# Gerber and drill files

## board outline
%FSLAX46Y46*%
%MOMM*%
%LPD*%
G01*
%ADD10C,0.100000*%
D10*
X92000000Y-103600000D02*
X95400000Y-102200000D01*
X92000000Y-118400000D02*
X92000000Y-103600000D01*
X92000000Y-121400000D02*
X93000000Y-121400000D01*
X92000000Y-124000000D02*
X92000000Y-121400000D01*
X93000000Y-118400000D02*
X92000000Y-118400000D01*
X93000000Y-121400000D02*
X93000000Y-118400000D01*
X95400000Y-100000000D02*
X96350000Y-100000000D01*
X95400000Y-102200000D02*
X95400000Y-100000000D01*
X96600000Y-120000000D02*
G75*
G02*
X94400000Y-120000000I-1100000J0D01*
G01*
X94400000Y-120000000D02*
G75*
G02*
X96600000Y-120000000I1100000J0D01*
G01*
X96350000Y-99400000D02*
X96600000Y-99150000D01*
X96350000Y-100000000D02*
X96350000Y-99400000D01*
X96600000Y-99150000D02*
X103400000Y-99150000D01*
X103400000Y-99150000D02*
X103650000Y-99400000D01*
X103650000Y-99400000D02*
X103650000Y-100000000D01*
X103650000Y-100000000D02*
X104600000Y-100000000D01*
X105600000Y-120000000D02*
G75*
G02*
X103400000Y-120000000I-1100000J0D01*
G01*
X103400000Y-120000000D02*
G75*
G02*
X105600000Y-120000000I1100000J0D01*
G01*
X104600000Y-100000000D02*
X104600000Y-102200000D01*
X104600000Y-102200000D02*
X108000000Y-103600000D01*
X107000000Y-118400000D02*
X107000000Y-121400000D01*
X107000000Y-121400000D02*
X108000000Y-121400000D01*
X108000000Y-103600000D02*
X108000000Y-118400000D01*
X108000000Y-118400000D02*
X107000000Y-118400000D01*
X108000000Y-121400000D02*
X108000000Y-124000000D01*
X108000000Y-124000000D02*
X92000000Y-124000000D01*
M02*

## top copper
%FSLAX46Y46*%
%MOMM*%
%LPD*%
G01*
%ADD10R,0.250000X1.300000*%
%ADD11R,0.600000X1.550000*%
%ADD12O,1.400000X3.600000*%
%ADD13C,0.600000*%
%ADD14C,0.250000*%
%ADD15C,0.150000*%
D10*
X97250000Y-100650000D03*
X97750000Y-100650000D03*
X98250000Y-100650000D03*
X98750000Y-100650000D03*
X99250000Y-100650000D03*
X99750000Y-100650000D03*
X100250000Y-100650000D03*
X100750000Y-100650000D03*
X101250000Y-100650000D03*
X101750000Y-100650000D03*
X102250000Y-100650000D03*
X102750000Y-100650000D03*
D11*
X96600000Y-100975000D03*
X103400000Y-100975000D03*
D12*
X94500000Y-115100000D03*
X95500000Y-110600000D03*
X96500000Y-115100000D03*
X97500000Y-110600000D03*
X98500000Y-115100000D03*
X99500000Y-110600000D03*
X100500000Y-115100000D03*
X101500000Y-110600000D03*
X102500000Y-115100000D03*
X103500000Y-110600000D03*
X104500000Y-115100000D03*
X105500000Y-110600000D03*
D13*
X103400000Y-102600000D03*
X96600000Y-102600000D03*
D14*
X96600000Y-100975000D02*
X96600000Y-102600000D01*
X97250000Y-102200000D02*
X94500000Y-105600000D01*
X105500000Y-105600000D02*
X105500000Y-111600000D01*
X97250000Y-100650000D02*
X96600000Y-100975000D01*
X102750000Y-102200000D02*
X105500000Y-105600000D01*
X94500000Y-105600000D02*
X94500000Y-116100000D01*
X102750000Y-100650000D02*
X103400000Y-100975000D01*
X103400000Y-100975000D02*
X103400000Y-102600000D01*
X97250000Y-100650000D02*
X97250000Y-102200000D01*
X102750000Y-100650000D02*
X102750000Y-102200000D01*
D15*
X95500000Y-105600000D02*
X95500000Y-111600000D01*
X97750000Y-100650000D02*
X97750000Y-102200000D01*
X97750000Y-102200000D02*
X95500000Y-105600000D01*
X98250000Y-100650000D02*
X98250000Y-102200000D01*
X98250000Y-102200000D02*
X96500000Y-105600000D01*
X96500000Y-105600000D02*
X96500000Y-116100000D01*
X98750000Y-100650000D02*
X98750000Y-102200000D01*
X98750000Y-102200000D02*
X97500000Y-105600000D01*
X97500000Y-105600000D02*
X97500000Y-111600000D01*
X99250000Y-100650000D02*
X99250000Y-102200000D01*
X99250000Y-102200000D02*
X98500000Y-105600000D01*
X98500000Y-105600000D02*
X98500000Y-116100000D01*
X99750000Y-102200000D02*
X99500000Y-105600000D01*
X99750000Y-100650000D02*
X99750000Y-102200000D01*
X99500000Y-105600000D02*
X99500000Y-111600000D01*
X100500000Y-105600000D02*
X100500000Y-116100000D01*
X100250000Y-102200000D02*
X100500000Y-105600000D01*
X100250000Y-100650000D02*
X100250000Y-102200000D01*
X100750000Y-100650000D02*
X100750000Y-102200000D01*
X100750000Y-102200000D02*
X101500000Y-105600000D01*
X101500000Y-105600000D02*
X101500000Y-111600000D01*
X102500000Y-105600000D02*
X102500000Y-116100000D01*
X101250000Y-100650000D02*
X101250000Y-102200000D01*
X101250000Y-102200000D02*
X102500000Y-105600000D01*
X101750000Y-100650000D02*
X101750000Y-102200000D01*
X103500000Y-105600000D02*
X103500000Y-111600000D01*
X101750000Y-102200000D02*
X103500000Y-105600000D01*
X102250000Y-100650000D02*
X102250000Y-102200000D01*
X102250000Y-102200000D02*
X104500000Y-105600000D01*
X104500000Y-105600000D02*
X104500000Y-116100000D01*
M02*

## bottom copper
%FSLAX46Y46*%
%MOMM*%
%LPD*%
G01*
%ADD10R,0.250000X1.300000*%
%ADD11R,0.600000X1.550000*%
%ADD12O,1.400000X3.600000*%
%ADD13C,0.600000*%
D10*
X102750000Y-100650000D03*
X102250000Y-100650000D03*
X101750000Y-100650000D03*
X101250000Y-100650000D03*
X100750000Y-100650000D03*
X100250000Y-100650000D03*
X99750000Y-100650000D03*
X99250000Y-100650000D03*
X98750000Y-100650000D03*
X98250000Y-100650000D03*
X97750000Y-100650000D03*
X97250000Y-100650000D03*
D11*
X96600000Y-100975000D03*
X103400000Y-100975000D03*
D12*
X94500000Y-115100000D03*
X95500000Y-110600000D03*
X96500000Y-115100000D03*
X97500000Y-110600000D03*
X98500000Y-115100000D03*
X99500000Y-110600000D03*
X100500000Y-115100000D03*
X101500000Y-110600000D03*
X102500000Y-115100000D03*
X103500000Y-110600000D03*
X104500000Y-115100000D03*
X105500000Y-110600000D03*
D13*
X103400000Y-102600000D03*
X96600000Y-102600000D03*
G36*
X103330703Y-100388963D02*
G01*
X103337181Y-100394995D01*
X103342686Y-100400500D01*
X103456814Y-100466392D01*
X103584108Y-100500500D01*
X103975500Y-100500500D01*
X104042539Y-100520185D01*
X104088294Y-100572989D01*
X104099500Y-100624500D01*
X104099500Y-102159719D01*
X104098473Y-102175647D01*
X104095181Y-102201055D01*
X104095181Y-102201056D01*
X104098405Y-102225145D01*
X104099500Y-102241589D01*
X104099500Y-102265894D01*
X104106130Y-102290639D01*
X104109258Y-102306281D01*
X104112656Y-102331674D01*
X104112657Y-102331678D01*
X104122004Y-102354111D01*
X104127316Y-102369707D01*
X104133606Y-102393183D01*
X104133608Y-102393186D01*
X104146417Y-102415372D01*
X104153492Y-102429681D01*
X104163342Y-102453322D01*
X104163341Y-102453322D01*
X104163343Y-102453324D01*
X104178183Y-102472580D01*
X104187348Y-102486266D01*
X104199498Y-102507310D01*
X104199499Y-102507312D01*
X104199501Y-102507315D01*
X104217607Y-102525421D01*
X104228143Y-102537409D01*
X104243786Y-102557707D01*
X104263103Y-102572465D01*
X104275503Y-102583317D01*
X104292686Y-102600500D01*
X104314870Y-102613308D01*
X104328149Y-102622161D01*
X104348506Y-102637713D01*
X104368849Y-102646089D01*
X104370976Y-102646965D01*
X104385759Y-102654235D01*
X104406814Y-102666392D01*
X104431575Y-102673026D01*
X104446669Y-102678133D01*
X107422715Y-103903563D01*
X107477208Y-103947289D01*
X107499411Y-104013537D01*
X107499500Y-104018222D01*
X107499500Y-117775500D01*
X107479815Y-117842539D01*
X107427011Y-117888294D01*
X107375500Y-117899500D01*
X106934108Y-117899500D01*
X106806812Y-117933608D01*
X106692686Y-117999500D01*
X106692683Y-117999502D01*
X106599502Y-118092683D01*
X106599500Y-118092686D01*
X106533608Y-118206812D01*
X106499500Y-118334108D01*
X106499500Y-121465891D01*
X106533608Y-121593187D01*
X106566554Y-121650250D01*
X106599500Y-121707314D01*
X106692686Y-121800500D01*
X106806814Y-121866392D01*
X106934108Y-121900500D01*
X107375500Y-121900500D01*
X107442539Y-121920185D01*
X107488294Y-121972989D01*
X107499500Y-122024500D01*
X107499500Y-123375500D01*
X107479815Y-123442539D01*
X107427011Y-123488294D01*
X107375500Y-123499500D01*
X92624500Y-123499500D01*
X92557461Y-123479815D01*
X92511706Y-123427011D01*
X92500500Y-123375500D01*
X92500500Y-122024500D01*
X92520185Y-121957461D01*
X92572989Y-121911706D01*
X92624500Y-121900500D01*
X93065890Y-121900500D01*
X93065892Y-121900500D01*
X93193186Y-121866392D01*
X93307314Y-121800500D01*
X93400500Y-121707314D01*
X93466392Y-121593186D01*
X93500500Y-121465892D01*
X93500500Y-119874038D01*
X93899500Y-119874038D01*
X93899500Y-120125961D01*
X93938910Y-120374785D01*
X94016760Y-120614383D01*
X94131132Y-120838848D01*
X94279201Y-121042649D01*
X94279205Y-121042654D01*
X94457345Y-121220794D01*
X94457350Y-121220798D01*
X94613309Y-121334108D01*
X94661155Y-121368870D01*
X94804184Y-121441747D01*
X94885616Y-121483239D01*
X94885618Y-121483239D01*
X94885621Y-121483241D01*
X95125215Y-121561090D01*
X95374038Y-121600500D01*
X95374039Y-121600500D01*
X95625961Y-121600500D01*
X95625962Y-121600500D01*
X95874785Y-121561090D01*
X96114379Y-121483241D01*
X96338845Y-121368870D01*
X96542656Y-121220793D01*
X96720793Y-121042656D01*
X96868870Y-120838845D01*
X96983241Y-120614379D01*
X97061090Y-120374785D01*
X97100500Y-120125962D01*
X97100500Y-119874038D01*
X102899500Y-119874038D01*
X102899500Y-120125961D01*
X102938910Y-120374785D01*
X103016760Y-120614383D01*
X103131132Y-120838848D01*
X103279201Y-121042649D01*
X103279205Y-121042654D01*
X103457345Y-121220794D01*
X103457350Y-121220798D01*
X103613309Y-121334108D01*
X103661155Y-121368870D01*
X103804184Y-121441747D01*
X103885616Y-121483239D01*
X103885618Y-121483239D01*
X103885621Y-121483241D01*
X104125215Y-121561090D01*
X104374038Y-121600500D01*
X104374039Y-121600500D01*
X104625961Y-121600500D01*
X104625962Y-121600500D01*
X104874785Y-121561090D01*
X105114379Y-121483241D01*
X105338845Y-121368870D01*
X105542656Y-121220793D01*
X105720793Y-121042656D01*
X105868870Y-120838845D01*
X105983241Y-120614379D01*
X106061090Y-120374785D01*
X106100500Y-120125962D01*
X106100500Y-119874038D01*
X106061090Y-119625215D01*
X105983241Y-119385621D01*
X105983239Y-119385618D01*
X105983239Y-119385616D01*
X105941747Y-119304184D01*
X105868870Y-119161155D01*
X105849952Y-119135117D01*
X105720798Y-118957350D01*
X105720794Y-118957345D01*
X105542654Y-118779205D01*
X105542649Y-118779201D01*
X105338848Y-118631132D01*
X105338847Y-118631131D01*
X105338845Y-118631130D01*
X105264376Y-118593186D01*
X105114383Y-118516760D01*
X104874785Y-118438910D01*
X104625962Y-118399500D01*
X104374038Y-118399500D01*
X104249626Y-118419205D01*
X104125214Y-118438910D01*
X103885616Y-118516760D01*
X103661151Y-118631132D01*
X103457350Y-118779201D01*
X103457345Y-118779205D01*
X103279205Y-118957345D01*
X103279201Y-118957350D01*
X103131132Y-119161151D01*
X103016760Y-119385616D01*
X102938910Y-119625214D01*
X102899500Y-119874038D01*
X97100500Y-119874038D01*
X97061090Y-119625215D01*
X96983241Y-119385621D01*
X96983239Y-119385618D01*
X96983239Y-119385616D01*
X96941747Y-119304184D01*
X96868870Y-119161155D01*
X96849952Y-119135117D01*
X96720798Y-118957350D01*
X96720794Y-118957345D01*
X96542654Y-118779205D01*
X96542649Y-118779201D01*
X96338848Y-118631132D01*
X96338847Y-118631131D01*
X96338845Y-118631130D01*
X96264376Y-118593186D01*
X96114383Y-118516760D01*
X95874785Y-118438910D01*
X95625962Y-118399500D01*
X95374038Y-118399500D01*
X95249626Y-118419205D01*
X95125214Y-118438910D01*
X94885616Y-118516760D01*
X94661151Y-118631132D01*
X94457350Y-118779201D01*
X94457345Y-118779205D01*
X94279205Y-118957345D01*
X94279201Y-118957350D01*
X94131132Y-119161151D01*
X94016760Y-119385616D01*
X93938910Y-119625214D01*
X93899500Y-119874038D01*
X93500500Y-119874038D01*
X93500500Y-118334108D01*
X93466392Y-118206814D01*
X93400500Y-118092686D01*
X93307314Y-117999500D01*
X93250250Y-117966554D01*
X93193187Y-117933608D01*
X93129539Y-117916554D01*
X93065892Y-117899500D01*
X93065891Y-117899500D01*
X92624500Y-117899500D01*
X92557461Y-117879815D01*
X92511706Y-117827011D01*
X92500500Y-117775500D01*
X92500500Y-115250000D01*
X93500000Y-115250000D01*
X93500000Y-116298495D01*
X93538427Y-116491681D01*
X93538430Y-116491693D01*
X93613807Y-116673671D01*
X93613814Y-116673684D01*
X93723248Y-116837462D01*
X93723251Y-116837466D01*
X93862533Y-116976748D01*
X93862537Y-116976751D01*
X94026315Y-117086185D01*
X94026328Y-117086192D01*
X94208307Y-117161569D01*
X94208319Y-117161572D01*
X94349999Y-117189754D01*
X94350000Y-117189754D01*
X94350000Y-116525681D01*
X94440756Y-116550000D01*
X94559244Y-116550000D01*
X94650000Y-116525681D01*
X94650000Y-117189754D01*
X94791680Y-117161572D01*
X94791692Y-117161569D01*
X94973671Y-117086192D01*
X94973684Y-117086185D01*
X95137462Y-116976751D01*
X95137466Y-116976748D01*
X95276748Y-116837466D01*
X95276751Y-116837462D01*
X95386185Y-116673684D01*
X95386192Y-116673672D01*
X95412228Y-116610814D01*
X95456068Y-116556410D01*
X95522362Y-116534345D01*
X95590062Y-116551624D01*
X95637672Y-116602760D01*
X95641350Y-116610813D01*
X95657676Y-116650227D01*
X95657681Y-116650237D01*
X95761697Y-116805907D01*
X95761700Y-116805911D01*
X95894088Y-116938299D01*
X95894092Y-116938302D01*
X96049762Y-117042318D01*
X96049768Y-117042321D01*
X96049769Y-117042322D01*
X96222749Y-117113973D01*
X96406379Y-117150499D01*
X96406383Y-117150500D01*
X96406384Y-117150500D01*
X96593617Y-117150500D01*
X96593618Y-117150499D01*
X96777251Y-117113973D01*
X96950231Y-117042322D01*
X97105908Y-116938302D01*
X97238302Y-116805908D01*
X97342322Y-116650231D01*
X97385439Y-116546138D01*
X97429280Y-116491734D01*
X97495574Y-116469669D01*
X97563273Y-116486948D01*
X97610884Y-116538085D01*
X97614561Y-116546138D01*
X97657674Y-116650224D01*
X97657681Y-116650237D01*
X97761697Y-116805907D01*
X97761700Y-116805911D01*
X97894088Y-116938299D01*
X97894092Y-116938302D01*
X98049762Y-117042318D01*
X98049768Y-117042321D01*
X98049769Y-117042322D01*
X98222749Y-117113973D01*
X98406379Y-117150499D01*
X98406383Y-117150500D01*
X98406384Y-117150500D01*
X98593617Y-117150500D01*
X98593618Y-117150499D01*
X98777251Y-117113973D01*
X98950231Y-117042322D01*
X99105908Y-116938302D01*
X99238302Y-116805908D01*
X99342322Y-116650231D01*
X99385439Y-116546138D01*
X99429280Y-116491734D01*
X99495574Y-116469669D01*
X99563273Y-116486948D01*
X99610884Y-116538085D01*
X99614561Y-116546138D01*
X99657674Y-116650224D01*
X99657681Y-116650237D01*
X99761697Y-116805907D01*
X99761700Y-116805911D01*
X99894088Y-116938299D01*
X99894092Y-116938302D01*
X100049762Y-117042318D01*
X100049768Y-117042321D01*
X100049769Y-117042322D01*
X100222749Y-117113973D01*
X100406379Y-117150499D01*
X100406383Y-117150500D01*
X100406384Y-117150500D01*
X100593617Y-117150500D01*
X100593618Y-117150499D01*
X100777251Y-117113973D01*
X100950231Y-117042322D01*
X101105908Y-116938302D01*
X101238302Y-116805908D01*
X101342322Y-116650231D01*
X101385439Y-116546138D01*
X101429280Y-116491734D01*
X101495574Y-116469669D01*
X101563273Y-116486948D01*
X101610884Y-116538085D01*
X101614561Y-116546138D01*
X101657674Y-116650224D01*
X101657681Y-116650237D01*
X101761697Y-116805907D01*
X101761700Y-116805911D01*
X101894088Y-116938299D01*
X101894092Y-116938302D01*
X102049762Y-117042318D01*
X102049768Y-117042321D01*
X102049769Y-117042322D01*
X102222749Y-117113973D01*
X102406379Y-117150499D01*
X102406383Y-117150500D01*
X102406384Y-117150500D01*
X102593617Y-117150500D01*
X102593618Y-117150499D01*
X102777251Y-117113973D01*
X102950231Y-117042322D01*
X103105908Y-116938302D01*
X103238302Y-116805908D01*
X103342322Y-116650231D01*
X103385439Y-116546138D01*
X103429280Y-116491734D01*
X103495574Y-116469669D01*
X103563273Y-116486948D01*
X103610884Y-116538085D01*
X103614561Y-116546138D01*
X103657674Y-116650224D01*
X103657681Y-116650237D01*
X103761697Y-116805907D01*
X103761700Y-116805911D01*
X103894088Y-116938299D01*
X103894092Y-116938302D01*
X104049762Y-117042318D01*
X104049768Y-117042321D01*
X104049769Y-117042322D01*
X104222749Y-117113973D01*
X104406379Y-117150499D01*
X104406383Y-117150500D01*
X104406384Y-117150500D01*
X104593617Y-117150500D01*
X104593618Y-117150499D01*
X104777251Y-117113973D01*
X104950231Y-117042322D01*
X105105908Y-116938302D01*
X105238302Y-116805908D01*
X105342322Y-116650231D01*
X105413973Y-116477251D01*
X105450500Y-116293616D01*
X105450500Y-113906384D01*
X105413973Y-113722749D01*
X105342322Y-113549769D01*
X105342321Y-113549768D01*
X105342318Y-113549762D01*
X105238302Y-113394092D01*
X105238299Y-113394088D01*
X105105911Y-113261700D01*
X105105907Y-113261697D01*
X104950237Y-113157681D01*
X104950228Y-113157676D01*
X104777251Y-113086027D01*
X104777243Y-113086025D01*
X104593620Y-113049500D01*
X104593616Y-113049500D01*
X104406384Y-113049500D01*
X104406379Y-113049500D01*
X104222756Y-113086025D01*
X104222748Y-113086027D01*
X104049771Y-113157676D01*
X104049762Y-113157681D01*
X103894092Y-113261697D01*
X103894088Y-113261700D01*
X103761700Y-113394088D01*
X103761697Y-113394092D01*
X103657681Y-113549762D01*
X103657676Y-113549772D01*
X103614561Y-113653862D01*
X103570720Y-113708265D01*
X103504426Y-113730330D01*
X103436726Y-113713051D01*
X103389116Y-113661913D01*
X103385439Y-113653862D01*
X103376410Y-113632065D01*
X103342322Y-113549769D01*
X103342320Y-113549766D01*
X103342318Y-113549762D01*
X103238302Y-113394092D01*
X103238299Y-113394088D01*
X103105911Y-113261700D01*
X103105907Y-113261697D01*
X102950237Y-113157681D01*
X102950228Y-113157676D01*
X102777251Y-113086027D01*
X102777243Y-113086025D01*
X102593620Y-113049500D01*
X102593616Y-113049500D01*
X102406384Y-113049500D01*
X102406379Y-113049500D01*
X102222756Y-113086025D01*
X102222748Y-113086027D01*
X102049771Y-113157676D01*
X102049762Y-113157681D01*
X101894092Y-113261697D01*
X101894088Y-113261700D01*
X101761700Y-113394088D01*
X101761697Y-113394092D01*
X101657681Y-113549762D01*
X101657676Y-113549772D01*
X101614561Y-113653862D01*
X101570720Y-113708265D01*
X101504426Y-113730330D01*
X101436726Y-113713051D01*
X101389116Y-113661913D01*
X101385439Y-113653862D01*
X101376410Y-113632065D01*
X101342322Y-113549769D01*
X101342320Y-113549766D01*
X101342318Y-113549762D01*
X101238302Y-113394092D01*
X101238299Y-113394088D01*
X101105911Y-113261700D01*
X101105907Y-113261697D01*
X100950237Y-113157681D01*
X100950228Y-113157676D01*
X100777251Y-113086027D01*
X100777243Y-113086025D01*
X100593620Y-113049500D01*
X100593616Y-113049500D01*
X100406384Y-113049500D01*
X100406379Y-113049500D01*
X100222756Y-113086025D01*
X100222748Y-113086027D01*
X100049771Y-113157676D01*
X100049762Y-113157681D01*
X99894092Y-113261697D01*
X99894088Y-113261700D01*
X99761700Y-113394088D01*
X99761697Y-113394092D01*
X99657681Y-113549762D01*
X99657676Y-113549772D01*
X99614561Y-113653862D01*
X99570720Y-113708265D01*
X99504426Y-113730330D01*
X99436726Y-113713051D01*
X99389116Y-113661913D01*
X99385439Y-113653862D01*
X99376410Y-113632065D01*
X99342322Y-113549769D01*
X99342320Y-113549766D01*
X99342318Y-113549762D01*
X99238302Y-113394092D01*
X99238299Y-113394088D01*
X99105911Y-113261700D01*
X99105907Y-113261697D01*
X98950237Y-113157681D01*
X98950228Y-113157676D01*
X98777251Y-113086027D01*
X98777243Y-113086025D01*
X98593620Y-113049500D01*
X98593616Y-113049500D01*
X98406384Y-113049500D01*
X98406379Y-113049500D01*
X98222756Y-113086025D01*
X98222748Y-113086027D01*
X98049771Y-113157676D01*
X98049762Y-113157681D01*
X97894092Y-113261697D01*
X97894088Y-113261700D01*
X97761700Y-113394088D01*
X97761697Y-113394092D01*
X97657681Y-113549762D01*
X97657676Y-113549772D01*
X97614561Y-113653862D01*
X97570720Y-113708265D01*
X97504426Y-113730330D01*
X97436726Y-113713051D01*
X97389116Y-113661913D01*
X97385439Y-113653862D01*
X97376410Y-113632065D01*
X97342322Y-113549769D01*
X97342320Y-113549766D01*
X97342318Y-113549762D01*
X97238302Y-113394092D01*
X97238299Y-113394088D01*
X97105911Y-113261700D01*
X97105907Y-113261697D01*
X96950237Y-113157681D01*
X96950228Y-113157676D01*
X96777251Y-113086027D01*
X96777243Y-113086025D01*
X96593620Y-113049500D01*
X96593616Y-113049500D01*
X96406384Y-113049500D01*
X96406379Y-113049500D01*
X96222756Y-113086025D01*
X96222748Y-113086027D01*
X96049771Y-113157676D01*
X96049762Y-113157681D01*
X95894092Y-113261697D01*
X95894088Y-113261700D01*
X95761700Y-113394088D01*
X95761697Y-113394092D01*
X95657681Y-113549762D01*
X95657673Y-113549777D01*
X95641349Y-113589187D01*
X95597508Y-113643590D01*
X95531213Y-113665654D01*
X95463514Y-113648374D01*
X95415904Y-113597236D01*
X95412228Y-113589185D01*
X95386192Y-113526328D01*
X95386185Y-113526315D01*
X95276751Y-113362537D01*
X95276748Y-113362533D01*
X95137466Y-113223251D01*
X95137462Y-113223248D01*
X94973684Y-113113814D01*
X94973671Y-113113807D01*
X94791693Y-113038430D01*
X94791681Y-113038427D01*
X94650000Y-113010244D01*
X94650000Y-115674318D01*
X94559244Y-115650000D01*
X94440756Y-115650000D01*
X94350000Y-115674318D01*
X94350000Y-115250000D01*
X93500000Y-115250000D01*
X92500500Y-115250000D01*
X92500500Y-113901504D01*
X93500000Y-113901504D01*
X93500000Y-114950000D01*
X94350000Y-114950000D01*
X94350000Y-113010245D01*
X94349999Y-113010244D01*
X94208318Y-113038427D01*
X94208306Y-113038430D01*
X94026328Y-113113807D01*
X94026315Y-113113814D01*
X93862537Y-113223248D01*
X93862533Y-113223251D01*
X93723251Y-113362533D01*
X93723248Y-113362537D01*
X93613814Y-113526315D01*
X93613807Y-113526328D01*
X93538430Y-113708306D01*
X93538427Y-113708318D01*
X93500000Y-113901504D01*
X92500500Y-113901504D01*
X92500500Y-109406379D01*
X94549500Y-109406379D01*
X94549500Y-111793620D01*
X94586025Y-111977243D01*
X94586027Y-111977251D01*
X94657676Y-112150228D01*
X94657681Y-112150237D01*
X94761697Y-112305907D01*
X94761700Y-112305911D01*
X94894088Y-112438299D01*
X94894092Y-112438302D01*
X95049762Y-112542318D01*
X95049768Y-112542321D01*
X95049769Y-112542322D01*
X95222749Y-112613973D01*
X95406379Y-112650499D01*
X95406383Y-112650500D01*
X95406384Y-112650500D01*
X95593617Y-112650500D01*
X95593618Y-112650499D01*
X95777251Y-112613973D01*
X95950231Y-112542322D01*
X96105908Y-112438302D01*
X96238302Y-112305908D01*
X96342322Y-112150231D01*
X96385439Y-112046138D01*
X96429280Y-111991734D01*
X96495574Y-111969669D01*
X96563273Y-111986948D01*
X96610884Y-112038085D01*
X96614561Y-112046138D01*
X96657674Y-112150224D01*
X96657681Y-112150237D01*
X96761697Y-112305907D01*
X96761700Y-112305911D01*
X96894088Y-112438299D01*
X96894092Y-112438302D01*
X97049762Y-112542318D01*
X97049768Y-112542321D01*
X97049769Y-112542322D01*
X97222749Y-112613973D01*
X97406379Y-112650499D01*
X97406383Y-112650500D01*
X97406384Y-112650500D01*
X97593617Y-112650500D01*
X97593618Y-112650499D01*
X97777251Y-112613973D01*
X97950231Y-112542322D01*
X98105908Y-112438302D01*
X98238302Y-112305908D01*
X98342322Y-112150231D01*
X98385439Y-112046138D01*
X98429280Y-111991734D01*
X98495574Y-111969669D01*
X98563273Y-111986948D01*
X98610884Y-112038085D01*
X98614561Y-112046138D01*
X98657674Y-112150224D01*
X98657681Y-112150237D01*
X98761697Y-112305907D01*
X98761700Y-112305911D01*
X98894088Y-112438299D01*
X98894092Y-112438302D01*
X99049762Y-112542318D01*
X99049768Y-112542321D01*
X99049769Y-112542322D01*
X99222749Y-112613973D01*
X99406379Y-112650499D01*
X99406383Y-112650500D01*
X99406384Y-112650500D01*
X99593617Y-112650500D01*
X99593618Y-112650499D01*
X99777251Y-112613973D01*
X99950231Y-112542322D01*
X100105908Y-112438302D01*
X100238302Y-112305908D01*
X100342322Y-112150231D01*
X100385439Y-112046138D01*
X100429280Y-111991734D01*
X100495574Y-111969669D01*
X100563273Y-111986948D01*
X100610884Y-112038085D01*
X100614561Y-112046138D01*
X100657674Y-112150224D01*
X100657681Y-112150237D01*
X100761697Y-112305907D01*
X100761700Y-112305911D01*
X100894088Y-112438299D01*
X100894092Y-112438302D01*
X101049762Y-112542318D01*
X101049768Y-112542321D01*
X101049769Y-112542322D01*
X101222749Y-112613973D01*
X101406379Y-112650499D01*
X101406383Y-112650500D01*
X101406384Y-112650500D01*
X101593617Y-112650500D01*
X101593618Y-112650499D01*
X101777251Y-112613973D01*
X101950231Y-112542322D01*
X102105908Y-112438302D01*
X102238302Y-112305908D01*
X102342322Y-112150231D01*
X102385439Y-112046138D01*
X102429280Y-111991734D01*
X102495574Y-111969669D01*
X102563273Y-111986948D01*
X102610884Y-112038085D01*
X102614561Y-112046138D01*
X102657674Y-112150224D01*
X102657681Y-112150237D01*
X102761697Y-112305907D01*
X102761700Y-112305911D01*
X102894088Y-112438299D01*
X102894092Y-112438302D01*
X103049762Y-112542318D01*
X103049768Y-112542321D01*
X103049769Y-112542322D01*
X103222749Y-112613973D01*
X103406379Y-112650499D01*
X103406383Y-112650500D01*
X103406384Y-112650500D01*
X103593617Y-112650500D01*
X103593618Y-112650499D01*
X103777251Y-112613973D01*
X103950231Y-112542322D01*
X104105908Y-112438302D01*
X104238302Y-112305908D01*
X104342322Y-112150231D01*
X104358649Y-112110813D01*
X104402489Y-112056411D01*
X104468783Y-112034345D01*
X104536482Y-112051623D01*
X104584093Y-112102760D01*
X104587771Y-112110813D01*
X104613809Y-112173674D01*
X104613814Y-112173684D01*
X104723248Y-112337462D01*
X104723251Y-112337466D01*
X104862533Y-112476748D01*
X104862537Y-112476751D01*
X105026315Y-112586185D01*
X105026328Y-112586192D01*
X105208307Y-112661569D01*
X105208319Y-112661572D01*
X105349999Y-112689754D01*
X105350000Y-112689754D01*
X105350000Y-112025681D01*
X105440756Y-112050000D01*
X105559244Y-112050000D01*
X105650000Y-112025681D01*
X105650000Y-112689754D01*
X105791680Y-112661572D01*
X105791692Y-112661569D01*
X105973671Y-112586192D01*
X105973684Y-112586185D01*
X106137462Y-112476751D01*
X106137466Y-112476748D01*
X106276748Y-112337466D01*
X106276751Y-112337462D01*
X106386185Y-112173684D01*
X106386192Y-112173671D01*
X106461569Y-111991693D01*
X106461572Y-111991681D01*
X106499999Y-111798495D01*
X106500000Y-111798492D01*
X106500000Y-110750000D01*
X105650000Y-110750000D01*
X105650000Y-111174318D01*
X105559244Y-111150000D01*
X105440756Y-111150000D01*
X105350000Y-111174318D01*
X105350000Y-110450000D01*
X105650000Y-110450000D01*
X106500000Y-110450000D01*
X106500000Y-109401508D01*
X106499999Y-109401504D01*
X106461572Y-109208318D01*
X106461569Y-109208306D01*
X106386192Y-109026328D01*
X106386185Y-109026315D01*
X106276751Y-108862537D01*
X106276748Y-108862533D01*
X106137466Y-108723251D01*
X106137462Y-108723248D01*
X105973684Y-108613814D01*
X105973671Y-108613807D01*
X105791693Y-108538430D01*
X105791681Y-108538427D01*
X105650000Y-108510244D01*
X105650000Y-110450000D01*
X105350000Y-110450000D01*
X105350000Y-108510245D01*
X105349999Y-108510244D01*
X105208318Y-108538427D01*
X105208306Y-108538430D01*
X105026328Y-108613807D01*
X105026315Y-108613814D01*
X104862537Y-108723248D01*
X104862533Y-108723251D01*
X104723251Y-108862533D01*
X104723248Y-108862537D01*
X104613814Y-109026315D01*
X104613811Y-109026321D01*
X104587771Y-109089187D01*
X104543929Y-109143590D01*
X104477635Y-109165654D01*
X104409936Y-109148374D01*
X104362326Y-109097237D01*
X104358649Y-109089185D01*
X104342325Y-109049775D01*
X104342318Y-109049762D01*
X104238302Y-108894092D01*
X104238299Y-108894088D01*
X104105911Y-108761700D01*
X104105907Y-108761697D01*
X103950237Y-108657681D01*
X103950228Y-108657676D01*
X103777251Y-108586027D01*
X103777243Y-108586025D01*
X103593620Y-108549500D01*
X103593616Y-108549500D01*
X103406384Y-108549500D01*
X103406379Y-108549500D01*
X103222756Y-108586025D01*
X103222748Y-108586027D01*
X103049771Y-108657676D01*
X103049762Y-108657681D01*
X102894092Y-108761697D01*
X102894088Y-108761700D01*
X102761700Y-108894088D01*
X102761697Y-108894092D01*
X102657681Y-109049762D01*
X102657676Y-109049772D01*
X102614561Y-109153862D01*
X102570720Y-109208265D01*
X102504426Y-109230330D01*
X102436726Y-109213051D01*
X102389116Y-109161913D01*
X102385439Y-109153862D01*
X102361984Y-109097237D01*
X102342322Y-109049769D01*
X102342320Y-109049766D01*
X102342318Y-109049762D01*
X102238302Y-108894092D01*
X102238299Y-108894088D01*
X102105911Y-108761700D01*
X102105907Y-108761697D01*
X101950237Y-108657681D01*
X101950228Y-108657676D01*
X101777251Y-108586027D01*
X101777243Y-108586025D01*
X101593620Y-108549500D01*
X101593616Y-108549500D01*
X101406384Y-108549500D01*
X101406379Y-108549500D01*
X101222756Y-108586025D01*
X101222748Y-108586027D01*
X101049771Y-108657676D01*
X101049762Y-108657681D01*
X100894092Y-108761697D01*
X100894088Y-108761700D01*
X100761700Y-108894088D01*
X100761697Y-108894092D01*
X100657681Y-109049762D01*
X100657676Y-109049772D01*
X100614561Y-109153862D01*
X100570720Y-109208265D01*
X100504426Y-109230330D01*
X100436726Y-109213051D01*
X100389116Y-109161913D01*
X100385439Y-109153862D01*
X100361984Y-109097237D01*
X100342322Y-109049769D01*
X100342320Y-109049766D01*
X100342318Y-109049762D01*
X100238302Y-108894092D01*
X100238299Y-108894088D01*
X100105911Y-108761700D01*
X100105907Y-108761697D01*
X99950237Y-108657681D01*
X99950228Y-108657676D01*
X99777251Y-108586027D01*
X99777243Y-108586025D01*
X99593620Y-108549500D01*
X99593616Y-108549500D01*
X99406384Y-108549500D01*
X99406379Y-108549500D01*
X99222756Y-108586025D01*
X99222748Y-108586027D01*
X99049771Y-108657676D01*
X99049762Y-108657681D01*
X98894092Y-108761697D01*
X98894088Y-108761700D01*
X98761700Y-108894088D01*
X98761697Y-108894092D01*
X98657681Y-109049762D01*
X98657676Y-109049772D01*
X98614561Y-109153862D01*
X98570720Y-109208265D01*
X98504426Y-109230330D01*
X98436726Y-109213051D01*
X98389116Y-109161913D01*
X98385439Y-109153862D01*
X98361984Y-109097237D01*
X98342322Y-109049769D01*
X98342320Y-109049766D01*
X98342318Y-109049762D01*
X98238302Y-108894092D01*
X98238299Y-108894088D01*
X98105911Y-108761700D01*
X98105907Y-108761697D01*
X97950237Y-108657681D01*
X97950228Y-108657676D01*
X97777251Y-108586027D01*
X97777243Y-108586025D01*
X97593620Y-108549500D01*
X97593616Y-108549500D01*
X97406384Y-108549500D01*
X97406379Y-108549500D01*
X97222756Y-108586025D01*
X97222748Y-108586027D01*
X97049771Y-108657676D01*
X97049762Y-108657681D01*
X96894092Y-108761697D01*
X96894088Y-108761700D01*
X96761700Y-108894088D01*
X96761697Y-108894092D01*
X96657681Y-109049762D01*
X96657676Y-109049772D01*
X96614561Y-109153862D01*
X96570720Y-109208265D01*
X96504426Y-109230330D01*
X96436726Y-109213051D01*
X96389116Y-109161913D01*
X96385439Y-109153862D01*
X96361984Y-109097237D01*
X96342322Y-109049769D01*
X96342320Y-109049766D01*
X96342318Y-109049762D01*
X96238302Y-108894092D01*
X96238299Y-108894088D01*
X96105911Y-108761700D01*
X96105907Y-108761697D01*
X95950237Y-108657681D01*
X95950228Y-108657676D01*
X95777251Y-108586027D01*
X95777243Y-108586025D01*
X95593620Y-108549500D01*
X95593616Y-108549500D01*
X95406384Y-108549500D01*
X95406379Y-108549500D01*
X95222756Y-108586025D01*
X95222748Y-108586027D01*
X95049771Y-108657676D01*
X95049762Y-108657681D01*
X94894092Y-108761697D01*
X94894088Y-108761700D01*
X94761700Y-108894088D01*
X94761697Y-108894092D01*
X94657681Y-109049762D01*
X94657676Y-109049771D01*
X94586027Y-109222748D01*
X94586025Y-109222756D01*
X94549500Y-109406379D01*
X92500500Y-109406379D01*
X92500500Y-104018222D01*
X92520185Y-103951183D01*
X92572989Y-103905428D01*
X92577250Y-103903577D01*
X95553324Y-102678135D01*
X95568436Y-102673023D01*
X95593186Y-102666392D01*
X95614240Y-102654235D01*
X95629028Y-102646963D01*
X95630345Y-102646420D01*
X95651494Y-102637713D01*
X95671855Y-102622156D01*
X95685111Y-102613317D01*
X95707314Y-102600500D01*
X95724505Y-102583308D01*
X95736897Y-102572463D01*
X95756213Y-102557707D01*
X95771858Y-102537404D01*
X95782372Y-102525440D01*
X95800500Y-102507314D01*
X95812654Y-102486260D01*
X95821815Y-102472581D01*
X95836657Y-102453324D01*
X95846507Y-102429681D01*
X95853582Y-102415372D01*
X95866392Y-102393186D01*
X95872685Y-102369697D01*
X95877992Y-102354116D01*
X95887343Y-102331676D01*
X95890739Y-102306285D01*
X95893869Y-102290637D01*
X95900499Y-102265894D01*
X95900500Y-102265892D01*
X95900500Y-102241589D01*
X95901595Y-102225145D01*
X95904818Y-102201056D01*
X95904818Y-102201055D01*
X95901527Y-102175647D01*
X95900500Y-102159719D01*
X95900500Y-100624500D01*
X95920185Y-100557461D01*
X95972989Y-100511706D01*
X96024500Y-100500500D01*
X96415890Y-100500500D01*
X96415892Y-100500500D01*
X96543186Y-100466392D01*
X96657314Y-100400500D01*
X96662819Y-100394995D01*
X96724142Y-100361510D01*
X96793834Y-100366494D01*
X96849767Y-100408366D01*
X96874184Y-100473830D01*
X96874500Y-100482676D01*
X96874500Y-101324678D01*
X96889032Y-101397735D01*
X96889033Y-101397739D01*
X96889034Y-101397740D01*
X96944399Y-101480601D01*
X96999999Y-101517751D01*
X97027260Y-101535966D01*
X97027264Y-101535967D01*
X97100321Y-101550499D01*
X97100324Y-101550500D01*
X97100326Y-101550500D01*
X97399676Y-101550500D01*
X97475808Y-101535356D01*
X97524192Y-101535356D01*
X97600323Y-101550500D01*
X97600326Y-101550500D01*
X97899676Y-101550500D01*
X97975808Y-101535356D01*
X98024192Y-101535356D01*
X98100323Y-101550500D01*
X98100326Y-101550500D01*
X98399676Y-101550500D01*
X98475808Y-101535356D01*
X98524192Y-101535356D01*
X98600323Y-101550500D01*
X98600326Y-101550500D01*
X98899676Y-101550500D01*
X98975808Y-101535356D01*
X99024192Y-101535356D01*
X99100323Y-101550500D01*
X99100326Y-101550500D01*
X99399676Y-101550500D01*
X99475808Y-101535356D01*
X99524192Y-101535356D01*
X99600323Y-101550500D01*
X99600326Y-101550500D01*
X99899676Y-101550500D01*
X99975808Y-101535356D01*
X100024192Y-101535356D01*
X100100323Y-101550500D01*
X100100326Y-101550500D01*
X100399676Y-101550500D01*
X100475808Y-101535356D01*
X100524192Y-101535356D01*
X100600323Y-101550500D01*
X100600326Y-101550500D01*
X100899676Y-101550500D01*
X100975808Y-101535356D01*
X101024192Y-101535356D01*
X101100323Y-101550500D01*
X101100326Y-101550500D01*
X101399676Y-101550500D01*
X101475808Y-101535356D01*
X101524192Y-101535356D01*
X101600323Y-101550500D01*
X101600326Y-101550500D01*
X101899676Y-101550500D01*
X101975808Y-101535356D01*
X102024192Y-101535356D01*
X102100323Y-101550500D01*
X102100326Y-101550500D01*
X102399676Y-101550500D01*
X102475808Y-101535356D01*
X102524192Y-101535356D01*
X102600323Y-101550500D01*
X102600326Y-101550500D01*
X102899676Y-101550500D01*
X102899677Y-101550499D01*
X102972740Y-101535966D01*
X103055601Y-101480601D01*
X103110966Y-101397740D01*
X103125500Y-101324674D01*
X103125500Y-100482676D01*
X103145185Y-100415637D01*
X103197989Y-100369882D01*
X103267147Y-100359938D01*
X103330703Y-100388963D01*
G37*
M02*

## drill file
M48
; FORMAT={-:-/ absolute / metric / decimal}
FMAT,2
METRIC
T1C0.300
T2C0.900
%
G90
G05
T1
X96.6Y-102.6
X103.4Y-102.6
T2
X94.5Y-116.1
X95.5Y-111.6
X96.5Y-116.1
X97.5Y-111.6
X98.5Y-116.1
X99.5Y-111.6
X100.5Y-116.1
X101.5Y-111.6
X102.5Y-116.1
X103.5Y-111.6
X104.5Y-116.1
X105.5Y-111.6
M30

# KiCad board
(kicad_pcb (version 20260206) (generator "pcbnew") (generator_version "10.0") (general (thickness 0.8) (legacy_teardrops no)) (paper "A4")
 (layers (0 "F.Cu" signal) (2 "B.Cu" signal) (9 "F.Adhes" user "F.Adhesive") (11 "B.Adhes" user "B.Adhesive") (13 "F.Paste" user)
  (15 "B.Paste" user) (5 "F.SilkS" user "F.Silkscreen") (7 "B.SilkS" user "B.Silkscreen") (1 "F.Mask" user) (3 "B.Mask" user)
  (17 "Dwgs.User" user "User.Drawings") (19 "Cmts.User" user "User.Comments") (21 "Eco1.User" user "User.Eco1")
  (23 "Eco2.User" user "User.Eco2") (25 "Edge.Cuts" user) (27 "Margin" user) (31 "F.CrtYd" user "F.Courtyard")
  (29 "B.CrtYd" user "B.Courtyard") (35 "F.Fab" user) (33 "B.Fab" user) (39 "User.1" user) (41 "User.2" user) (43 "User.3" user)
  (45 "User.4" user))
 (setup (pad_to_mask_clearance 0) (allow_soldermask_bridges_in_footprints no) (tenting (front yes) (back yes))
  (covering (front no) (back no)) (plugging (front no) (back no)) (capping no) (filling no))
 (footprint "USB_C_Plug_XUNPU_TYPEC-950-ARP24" (layer "F.Cu") (at 100 100)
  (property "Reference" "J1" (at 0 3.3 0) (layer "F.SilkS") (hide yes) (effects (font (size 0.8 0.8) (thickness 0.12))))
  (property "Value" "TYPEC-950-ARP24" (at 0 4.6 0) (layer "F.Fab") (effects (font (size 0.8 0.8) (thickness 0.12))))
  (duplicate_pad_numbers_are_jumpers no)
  (pad "A1" smd rect (at -2.75 0.65) (size 0.25 1.3) (layers "F.Cu" "F.Mask" "F.Paste") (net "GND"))
  (pad "A2" smd rect (at -2.25 0.65) (size 0.25 1.3) (layers "F.Cu" "F.Mask" "F.Paste") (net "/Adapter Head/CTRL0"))
  (pad "A3" smd rect (at -1.75 0.65) (size 0.25 1.3) (layers "F.Cu" "F.Mask" "F.Paste") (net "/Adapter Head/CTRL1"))
  (pad "A4" smd rect (at -1.25 0.65) (size 0.25 1.3) (layers "F.Cu" "F.Mask" "F.Paste") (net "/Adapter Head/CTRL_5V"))
  (pad "A5" smd rect (at -0.75 0.65) (size 0.25 1.3) (layers "F.Cu" "F.Mask" "F.Paste") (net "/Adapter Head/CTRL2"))
  (pad "A6" smd rect (at -0.25 0.65) (size 0.25 1.3) (layers "F.Cu" "F.Mask" "F.Paste") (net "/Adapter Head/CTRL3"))
  (pad "A7" smd rect (at 0.25 0.65) (size 0.25 1.3) (layers "F.Cu" "F.Mask" "F.Paste") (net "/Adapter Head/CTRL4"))
  (pad "A8" smd rect (at 0.75 0.65) (size 0.25 1.3) (layers "F.Cu" "F.Mask" "F.Paste") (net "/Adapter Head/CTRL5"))
  (pad "A9" smd rect (at 1.25 0.65) (size 0.25 1.3) (layers "F.Cu" "F.Mask" "F.Paste") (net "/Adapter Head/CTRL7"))
  (pad "A10" smd rect (at 1.75 0.65) (size 0.25 1.3) (layers "F.Cu" "F.Mask" "F.Paste") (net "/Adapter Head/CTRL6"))
  (pad "A11" smd rect (at 2.25 0.65) (size 0.25 1.3) (layers "F.Cu" "F.Mask" "F.Paste") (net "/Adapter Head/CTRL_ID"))
  (pad "A12" smd rect (at 2.75 0.65) (size 0.25 1.3) (layers "F.Cu" "F.Mask" "F.Paste") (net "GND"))
  (pad "B1" smd rect (at 2.75 0.65) (size 0.25 1.3) (layers "B.Cu" "B.Mask" "B.Paste") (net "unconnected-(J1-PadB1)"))
  (pad "B2" smd rect (at 2.25 0.65) (size 0.25 1.3) (layers "B.Cu" "B.Mask" "B.Paste") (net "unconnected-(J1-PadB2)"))
  (pad "B3" smd rect (at 1.75 0.65) (size 0.25 1.3) (layers "B.Cu" "B.Mask" "B.Paste") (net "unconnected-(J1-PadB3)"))
  (pad "B4" smd rect (at 1.25 0.65) (size 0.25 1.3) (layers "B.Cu" "B.Mask" "B.Paste") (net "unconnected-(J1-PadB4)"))
  (pad "B5" smd rect (at 0.75 0.65) (size 0.25 1.3) (layers "B.Cu" "B.Mask" "B.Paste") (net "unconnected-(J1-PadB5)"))
  (pad "B6" smd rect (at 0.25 0.65) (size 0.25 1.3) (layers "B.Cu" "B.Mask" "B.Paste") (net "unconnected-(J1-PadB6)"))
  (pad "B7" smd rect (at -0.25 0.65) (size 0.25 1.3) (layers "B.Cu" "B.Mask" "B.Paste") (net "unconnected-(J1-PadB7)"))
  (pad "B8" smd rect (at -0.75 0.65) (size 0.25 1.3) (layers "B.Cu" "B.Mask" "B.Paste") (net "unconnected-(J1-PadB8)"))
  (pad "B9" smd rect (at -1.25 0.65) (size 0.25 1.3) (layers "B.Cu" "B.Mask" "B.Paste") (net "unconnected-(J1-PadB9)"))
  (pad "B10" smd rect (at -1.75 0.65) (size 0.25 1.3) (layers "B.Cu" "B.Mask" "B.Paste") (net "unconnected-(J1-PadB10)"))
  (pad "B11" smd rect (at -2.25 0.65) (size 0.25 1.3) (layers "B.Cu" "B.Mask" "B.Paste") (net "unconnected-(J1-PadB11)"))
  (pad "B12" smd rect (at -2.75 0.65) (size 0.25 1.3) (layers "B.Cu" "B.Mask" "B.Paste") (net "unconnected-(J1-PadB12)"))
  (pad "SH" smd rect (at -3.4 0.975) (size 0.6 1.55) (layers "F.Cu" "F.Mask" "F.Paste") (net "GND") (zone_connect 2))
  (pad "SH" smd rect (at -3.4 0.975) (size 0.6 1.55) (layers "B.Cu" "B.Mask" "B.Paste") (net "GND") (zone_connect 2))
  (pad "SH" smd rect (at 3.4 0.975) (size 0.6 1.55) (layers "F.Cu" "F.Mask" "F.Paste") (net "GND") (zone_connect 2))
  (pad "SH" smd rect (at 3.4 0.975) (size 0.6 1.55) (layers "B.Cu" "B.Mask" "B.Paste") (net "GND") (zone_connect 2)))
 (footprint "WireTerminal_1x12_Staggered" (layer "F.Cu") (at 100 111.6)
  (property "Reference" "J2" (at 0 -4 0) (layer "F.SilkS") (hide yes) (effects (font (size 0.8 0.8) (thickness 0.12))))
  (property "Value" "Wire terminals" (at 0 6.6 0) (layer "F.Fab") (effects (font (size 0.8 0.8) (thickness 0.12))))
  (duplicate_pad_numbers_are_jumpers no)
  (pad "1" thru_hole oval (at -5.5 4.5) (size 1.4 3.6) (drill 0.9 (offset 0 -1)) (layers "*.Cu" "*.Mask") (remove_unused_layers no)
   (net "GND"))
  (pad "2" thru_hole oval (at -4.5 0) (size 1.4 3.6) (drill 0.9 (offset 0 -1)) (layers "*.Cu" "*.Mask") (remove_unused_layers no)
   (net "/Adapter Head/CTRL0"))
  (pad "3" thru_hole oval (at -3.5 4.5) (size 1.4 3.6) (drill 0.9 (offset 0 -1)) (layers "*.Cu" "*.Mask") (remove_unused_layers no)
   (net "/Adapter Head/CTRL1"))
  (pad "4" thru_hole oval (at -2.5 0) (size 1.4 3.6) (drill 0.9 (offset 0 -1)) (layers "*.Cu" "*.Mask") (remove_unused_layers no)
   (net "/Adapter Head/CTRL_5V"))
  (pad "5" thru_hole oval (at -1.5 4.5) (size 1.4 3.6) (drill 0.9 (offset 0 -1)) (layers "*.Cu" "*.Mask") (remove_unused_layers no)
   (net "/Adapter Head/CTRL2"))
  (pad "6" thru_hole oval (at -0.5 0) (size 1.4 3.6) (drill 0.9 (offset 0 -1)) (layers "*.Cu" "*.Mask") (remove_unused_layers no)
   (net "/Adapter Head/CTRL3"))
  (pad "7" thru_hole oval (at 0.5 4.5) (size 1.4 3.6) (drill 0.9 (offset 0 -1)) (layers "*.Cu" "*.Mask") (remove_unused_layers no)
   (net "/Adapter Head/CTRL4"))
  (pad "8" thru_hole oval (at 1.5 0) (size 1.4 3.6) (drill 0.9 (offset 0 -1)) (layers "*.Cu" "*.Mask") (remove_unused_layers no)
   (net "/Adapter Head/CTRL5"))
  (pad "9" thru_hole oval (at 2.5 4.5) (size 1.4 3.6) (drill 0.9 (offset 0 -1)) (layers "*.Cu" "*.Mask") (remove_unused_layers no)
   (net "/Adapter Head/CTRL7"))
  (pad "10" thru_hole oval (at 3.5 0) (size 1.4 3.6) (drill 0.9 (offset 0 -1)) (layers "*.Cu" "*.Mask") (remove_unused_layers no)
   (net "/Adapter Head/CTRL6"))
  (pad "11" thru_hole oval (at 4.5 4.5) (size 1.4 3.6) (drill 0.9 (offset 0 -1)) (layers "*.Cu" "*.Mask") (remove_unused_layers no)
   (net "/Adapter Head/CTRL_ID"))
  (pad "12" thru_hole oval (at 5.5 0) (size 1.4 3.6) (drill 0.9 (offset 0 -1)) (layers "*.Cu" "*.Mask") (remove_unused_layers no)
   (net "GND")))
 (gr_line (start 92 103.6) (end 95.4 102.2) (stroke (width 0.1) (type default)) (layer "Edge.Cuts"))
 (gr_line (start 92 118.4) (end 92 103.6) (stroke (width 0.1) (type default)) (layer "Edge.Cuts"))
 (gr_line (start 92 121.4) (end 93 121.4) (stroke (width 0.1) (type default)) (layer "Edge.Cuts"))
 (gr_line (start 92 124) (end 92 121.4) (stroke (width 0.1) (type default)) (layer "Edge.Cuts"))
 (gr_line (start 93 118.4) (end 92 118.4) (stroke (width 0.1) (type default)) (layer "Edge.Cuts"))
 (gr_line (start 93 121.4) (end 93 118.4) (stroke (width 0.1) (type default)) (layer "Edge.Cuts"))
 (gr_line (start 95.4 100) (end 96.35 100) (stroke (width 0.1) (type default)) (layer "Edge.Cuts"))
 (gr_line (start 95.4 102.2) (end 95.4 100) (stroke (width 0.1) (type default)) (layer "Edge.Cuts"))
 (gr_circle (center 95.5 120) (end 96.6 120) (stroke (width 0.1) (type default)) (fill no) (layer "Edge.Cuts"))
 (gr_line (start 96.35 99.4) (end 96.6 99.15) (stroke (width 0.1) (type default)) (layer "Edge.Cuts"))
 (gr_line (start 96.35 100) (end 96.35 99.4) (stroke (width 0.1) (type default)) (layer "Edge.Cuts"))
 (gr_line (start 96.6 99.15) (end 103.4 99.15) (stroke (width 0.1) (type default)) (layer "Edge.Cuts"))
 (gr_line (start 103.4 99.15) (end 103.65 99.4) (stroke (width 0.1) (type default)) (layer "Edge.Cuts"))
 (gr_line (start 103.65 99.4) (end 103.65 100) (stroke (width 0.1) (type default)) (layer "Edge.Cuts"))
 (gr_line (start 103.65 100) (end 104.6 100) (stroke (width 0.1) (type default)) (layer "Edge.Cuts"))
 (gr_circle (center 104.5 120) (end 105.6 120) (stroke (width 0.1) (type default)) (fill no) (layer "Edge.Cuts"))
 (gr_line (start 104.6 100) (end 104.6 102.2) (stroke (width 0.1) (type default)) (layer "Edge.Cuts"))
 (gr_line (start 104.6 102.2) (end 108 103.6) (stroke (width 0.1) (type default)) (layer "Edge.Cuts"))
 (gr_line (start 107 118.4) (end 107 121.4) (stroke (width 0.1) (type default)) (layer "Edge.Cuts"))
 (gr_line (start 107 121.4) (end 108 121.4) (stroke (width 0.1) (type default)) (layer "Edge.Cuts"))
 (gr_line (start 108 103.6) (end 108 118.4) (stroke (width 0.1) (type default)) (layer "Edge.Cuts"))
 (gr_line (start 108 118.4) (end 107 118.4) (stroke (width 0.1) (type default)) (layer "Edge.Cuts"))
 (gr_line (start 108 121.4) (end 108 124) (stroke (width 0.1) (type default)) (layer "Edge.Cuts"))
 (gr_line (start 108 124) (end 92 124) (stroke (width 0.1) (type default)) (layer "Edge.Cuts"))
 (segment (start 96.6 100.975) (end 96.6 102.6) (width 0.25) (layer "F.Cu") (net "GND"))
 (segment (start 97.25 102.2) (end 94.5 105.6) (width 0.25) (layer "F.Cu") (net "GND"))
 (segment (start 105.5 105.6) (end 105.5 111.6) (width 0.25) (layer "F.Cu") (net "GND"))
 (segment (start 97.25 100.65) (end 96.6 100.975) (width 0.25) (layer "F.Cu") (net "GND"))
 (segment (start 102.75 102.2) (end 105.5 105.6) (width 0.25) (layer "F.Cu") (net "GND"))
 (segment (start 94.5 105.6) (end 94.5 116.1) (width 0.25) (layer "F.Cu") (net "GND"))
 (segment (start 102.75 100.65) (end 103.4 100.975) (width 0.25) (layer "F.Cu") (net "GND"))
 (segment (start 103.4 100.975) (end 103.4 102.6) (width 0.25) (layer "F.Cu") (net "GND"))
 (segment (start 97.25 100.65) (end 97.25 102.2) (width 0.25) (layer "F.Cu") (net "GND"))
 (segment (start 102.75 100.65) (end 102.75 102.2) (width 0.25) (layer "F.Cu") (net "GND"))
 (via (at 103.4 102.6) (size 0.6) (drill 0.3) (layers "F.Cu" "B.Cu") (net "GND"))
 (via (at 96.6 102.6) (size 0.6) (drill 0.3) (layers "F.Cu" "B.Cu") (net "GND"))
 (segment (start 95.5 105.6) (end 95.5 111.6) (width 0.15) (layer "F.Cu") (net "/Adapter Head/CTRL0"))
 (segment (start 97.75 100.65) (end 97.75 102.2) (width 0.15) (layer "F.Cu") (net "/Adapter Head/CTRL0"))
 (segment (start 97.75 102.2) (end 95.5 105.6) (width 0.15) (layer "F.Cu") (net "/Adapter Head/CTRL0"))
 (segment (start 98.25 100.65) (end 98.25 102.2) (width 0.15) (layer "F.Cu") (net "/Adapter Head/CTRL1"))
 (segment (start 98.25 102.2) (end 96.5 105.6) (width 0.15) (layer "F.Cu") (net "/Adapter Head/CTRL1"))
 (segment (start 96.5 105.6) (end 96.5 116.1) (width 0.15) (layer "F.Cu") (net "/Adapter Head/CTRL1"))
 (segment (start 98.75 100.65) (end 98.75 102.2) (width 0.15) (layer "F.Cu") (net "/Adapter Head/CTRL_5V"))
 (segment (start 98.75 102.2) (end 97.5 105.6) (width 0.15) (layer "F.Cu") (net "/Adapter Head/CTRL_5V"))
 (segment (start 97.5 105.6) (end 97.5 111.6) (width 0.15) (layer "F.Cu") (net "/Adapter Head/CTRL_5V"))
 (segment (start 99.25 100.65) (end 99.25 102.2) (width 0.15) (layer "F.Cu") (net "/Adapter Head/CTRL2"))
 (segment (start 99.25 102.2) (end 98.5 105.6) (width 0.15) (layer "F.Cu") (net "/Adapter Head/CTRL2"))
 (segment (start 98.5 105.6) (end 98.5 116.1) (width 0.15) (layer "F.Cu") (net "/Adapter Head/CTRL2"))
 (segment (start 99.75 102.2) (end 99.5 105.6) (width 0.15) (layer "F.Cu") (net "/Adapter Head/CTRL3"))
 (segment (start 99.75 100.65) (end 99.75 102.2) (width 0.15) (layer "F.Cu") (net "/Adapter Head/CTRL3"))
 (segment (start 99.5 105.6) (end 99.5 111.6) (width 0.15) (layer "F.Cu") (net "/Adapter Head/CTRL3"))
 (segment (start 100.5 105.6) (end 100.5 116.1) (width 0.15) (layer "F.Cu") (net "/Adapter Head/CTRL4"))
 (segment (start 100.25 102.2) (end 100.5 105.6) (width 0.15) (layer "F.Cu") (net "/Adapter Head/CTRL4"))
 (segment (start 100.25 100.65) (end 100.25 102.2) (width 0.15) (layer "F.Cu") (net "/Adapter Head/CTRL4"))
 (segment (start 100.75 100.65) (end 100.75 102.2) (width 0.15) (layer "F.Cu") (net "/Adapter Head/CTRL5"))
 (segment (start 100.75 102.2) (end 101.5 105.6) (width 0.15) (layer "F.Cu") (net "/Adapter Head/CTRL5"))
 (segment (start 101.5 105.6) (end 101.5 111.6) (width 0.15) (layer "F.Cu") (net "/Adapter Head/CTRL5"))
 (segment (start 102.5 105.6) (end 102.5 116.1) (width 0.15) (layer "F.Cu") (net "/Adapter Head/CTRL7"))
 (segment (start 101.25 100.65) (end 101.25 102.2) (width 0.15) (layer "F.Cu") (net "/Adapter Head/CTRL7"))
 (segment (start 101.25 102.2) (end 102.5 105.6) (width 0.15) (layer "F.Cu") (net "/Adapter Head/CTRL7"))
 (segment (start 101.75 100.65) (end 101.75 102.2) (width 0.15) (layer "F.Cu") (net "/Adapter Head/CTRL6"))
 (segment (start 103.5 105.6) (end 103.5 111.6) (width 0.15) (layer "F.Cu") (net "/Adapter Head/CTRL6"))
 (segment (start 101.75 102.2) (end 103.5 105.6) (width 0.15) (layer "F.Cu") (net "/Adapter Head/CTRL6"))
 (segment (start 102.25 100.65) (end 102.25 102.2) (width 0.15) (layer "F.Cu") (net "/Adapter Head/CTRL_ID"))
 (segment (start 102.25 102.2) (end 104.5 105.6) (width 0.15) (layer "F.Cu") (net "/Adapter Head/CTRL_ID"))
 (segment (start 104.5 105.6) (end 104.5 116.1) (width 0.15) (layer "F.Cu") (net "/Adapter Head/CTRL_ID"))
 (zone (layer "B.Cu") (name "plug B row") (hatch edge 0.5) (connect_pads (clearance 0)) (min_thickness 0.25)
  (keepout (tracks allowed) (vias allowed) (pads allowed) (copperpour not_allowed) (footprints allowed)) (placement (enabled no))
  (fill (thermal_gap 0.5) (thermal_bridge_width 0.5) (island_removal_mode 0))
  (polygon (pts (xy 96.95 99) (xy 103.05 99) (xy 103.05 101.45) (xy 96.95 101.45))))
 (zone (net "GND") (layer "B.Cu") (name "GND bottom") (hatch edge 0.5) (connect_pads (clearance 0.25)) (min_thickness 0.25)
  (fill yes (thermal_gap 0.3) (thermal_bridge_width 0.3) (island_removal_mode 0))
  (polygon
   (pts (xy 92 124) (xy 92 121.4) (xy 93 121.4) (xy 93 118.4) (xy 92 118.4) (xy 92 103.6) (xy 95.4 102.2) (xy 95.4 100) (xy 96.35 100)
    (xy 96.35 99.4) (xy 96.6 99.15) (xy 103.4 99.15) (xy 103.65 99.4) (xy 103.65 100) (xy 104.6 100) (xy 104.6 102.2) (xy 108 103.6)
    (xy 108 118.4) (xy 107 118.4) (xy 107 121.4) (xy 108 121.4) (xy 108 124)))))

